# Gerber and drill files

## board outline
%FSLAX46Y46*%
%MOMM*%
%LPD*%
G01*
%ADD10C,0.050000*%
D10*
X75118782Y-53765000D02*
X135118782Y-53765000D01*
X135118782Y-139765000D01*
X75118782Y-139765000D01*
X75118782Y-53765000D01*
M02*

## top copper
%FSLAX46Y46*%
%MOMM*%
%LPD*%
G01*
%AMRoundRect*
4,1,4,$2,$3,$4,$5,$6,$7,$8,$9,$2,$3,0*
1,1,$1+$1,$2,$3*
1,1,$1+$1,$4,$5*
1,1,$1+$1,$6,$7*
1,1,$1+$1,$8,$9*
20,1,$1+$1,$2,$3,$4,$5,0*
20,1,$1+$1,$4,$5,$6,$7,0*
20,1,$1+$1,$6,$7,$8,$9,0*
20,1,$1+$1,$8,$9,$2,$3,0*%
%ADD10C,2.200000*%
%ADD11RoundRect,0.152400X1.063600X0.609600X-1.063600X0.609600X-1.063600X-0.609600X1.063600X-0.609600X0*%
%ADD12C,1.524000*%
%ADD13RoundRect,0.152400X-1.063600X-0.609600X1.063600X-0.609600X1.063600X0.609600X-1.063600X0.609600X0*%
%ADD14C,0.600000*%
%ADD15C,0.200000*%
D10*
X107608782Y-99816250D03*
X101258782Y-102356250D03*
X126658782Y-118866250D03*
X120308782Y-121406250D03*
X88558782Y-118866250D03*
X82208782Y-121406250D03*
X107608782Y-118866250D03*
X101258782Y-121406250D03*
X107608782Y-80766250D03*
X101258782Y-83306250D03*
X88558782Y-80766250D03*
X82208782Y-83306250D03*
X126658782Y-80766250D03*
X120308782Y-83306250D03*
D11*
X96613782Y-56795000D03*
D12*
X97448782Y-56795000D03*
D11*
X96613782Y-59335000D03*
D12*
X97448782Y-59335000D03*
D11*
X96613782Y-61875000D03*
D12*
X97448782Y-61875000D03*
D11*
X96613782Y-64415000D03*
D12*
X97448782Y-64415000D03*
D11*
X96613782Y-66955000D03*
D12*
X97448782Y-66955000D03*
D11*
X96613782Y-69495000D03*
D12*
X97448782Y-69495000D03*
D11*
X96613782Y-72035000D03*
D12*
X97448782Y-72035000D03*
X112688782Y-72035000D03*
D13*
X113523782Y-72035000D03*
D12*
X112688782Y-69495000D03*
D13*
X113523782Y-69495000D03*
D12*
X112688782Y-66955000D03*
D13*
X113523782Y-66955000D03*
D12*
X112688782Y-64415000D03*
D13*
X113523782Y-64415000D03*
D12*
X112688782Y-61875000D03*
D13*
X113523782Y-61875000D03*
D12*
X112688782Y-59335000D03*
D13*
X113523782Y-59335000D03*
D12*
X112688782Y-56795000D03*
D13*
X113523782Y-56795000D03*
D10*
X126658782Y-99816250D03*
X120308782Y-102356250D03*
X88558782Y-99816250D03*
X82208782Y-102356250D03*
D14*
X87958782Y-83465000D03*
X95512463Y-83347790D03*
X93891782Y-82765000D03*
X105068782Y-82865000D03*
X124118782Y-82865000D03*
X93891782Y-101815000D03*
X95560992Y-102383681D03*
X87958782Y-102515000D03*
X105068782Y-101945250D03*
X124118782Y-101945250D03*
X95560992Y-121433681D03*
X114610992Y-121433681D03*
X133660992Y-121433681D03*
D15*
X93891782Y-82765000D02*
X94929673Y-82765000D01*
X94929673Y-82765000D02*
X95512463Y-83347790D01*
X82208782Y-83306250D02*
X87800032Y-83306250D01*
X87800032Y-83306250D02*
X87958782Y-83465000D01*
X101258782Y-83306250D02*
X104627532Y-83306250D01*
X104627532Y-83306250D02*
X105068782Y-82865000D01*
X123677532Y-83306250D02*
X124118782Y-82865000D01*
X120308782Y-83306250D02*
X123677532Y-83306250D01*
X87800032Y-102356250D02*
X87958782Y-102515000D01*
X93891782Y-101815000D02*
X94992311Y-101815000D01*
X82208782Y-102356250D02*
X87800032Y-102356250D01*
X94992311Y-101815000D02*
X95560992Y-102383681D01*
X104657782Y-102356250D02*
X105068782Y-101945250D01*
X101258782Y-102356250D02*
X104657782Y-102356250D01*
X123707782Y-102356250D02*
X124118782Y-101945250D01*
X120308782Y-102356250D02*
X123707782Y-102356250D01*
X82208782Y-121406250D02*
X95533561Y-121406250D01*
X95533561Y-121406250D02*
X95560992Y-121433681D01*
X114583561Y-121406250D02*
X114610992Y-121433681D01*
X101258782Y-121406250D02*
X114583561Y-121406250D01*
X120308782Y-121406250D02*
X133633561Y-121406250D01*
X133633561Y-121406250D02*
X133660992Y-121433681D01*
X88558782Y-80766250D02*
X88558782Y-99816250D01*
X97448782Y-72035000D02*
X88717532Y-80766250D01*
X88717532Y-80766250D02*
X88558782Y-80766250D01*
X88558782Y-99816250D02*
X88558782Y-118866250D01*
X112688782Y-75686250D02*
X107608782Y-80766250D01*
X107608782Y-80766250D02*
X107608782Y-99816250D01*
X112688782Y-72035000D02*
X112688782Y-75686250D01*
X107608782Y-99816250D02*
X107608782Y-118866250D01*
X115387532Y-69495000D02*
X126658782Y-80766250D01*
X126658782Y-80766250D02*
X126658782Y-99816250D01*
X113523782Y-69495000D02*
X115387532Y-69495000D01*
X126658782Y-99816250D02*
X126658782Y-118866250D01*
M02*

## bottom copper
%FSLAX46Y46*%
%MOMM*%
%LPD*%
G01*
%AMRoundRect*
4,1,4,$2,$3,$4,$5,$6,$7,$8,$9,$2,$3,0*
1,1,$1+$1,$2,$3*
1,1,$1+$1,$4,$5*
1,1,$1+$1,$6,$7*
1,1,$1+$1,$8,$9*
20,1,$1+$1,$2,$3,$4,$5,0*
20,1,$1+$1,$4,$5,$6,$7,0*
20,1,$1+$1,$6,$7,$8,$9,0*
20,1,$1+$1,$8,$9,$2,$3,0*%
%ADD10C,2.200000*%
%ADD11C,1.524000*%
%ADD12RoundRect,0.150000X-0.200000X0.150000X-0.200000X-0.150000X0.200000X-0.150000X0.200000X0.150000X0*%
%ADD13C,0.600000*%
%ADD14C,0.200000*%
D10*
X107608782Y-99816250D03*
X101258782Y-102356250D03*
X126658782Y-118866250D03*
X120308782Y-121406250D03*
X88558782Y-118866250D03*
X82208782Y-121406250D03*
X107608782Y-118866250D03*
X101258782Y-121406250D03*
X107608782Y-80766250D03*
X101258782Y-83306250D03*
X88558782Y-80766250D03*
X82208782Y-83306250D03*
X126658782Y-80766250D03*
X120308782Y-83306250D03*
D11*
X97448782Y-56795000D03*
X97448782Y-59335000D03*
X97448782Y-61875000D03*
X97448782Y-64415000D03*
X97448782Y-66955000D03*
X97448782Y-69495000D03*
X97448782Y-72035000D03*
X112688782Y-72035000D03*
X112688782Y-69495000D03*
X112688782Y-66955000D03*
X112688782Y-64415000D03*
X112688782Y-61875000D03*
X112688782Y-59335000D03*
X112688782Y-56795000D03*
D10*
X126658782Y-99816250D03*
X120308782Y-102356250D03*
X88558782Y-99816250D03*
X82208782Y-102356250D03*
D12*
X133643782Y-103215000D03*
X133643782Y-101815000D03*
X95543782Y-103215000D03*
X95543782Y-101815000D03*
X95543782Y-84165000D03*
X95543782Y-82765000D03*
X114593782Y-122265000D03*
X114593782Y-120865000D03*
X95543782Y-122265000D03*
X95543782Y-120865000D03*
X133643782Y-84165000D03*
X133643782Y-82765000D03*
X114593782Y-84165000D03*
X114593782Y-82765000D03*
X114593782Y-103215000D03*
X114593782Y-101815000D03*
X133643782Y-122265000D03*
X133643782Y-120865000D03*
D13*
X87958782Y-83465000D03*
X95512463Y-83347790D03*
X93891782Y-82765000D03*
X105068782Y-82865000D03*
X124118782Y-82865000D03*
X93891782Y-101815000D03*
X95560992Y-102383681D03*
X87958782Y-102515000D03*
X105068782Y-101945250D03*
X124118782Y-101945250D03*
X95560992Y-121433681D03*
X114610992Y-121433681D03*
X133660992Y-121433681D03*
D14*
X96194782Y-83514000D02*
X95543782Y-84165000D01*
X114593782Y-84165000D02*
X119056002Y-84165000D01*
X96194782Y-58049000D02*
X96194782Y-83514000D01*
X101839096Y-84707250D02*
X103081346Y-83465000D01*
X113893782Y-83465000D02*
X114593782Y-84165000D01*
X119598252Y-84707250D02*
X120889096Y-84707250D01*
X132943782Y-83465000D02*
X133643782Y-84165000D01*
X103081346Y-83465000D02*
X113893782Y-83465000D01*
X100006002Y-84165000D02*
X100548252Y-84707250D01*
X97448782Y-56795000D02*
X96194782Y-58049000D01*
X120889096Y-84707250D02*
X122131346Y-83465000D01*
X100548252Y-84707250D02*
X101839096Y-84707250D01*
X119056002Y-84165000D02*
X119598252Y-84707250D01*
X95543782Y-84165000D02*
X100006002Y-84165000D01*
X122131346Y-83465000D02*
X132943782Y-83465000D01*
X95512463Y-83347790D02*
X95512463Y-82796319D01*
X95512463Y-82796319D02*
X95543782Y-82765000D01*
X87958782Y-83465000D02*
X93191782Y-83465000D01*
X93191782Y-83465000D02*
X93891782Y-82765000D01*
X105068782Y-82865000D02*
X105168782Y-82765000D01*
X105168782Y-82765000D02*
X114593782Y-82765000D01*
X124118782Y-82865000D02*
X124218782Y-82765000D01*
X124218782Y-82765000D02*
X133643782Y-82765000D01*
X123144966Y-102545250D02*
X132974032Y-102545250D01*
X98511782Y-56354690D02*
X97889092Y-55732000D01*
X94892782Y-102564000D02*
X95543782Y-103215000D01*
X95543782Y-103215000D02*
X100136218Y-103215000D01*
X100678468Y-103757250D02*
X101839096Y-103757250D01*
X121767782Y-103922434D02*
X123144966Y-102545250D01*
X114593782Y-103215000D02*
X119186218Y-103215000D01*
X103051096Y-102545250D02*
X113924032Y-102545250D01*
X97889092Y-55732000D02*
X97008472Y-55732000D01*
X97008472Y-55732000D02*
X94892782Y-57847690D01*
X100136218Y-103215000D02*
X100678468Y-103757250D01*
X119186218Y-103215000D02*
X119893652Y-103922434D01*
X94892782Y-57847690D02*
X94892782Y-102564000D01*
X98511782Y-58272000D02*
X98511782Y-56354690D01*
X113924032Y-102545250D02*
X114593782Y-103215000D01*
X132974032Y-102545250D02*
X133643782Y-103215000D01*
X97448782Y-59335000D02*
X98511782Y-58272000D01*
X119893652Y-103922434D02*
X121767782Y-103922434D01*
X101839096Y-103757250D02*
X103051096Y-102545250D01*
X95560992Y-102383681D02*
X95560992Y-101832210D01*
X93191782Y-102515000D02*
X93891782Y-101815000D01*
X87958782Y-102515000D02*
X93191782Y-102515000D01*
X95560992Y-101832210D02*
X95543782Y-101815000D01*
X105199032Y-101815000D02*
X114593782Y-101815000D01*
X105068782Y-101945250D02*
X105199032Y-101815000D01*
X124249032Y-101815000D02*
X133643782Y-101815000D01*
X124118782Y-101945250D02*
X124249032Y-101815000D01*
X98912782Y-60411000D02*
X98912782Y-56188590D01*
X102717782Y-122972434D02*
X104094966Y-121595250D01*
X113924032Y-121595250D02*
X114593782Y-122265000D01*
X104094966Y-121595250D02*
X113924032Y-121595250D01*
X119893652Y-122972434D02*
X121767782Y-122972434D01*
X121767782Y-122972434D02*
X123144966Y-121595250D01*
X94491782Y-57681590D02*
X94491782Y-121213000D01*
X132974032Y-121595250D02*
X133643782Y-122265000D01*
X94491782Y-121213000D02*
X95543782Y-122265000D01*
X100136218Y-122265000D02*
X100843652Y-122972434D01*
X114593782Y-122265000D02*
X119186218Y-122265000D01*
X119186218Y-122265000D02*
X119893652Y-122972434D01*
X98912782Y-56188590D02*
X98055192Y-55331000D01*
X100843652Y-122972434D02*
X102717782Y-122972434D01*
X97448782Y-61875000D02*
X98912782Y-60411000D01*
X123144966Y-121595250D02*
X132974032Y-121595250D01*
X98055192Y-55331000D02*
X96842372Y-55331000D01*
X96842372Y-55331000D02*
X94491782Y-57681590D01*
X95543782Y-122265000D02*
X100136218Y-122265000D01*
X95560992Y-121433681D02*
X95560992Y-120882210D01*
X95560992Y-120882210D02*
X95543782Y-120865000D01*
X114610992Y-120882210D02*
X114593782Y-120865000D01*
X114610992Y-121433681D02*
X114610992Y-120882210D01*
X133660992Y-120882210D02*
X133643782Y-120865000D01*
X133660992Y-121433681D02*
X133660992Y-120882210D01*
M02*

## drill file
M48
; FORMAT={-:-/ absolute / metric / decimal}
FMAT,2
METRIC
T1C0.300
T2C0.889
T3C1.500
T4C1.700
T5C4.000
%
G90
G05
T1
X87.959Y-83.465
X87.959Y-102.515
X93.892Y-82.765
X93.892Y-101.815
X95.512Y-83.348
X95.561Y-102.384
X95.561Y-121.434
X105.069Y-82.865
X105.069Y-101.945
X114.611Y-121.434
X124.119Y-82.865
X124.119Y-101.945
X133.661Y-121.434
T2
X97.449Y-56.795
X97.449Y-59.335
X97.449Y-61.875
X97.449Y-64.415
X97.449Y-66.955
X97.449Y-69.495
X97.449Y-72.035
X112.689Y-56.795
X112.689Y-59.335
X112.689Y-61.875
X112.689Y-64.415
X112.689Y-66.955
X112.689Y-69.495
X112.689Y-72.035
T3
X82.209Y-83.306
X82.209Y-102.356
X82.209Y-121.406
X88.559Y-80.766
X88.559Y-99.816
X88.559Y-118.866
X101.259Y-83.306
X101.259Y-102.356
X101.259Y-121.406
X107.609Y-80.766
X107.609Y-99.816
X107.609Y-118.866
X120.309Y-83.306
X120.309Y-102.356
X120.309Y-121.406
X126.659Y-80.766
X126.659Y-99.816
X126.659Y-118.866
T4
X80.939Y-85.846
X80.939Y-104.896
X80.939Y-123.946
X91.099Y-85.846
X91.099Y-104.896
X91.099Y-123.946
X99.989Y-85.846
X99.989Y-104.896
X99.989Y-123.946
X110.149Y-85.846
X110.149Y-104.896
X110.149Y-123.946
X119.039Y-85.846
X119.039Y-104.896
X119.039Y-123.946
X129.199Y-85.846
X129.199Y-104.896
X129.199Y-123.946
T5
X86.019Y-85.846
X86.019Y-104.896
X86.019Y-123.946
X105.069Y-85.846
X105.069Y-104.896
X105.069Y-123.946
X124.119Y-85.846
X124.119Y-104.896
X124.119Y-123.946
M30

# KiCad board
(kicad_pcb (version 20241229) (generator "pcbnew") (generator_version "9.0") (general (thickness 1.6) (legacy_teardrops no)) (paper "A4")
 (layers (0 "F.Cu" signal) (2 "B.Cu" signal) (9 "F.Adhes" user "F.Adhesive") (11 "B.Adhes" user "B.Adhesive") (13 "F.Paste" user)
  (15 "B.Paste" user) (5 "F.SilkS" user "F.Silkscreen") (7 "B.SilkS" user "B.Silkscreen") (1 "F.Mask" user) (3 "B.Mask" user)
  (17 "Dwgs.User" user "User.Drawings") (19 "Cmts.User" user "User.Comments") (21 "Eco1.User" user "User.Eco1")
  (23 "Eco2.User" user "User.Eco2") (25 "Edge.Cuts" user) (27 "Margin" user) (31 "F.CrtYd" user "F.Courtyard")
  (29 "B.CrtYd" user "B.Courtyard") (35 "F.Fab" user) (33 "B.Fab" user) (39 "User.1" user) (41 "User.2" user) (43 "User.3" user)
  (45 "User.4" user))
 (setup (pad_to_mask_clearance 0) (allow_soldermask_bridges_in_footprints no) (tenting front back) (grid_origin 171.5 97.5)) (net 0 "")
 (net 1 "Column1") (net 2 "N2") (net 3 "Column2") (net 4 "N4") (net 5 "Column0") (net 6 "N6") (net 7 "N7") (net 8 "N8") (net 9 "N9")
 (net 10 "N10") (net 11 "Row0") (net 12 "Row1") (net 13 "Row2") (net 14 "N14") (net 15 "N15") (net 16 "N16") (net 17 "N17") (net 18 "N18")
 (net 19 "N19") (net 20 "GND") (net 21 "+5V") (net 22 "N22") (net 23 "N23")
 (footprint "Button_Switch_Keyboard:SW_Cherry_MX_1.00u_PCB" (layer "F.Cu") (at 107.608782 99.81625)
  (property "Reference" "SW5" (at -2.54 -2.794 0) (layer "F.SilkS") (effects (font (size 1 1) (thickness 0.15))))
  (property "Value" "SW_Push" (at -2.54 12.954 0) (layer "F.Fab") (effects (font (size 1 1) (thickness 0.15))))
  (pad "" np_thru_hole circle (at -7.62 5.08) (size 1.7 1.7) (drill 1.7) (layers "*.Cu" "*.Mask"))
  (pad "" np_thru_hole circle (at -2.54 5.08) (size 4 4) (drill 4) (layers "*.Cu" "*.Mask"))
  (pad "" np_thru_hole circle (at 2.54 5.08) (size 1.7 1.7) (drill 1.7) (layers "*.Cu" "*.Mask"))
  (pad "1" thru_hole circle (at 0 0) (size 2.2 2.2) (drill 1.5) (layers "*.Cu" "*.Mask") (remove_unused_layers no) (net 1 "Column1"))
  (pad "2" thru_hole circle (at -6.35 2.54) (size 2.2 2.2) (drill 1.5) (layers "*.Cu" "*.Mask") (remove_unused_layers no) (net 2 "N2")))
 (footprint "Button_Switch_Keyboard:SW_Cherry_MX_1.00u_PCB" (layer "F.Cu") (at 126.658782 118.86625)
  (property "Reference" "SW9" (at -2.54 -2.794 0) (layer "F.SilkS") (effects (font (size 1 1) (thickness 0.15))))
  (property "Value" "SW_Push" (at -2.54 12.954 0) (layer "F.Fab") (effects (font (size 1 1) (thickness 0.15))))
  (pad "" np_thru_hole circle (at -7.62 5.08) (size 1.7 1.7) (drill 1.7) (layers "*.Cu" "*.Mask"))
  (pad "" np_thru_hole circle (at -2.54 5.08) (size 4 4) (drill 4) (layers "*.Cu" "*.Mask"))
  (pad "" np_thru_hole circle (at 2.54 5.08) (size 1.7 1.7) (drill 1.7) (layers "*.Cu" "*.Mask"))
  (pad "1" thru_hole circle (at 0 0) (size 2.2 2.2) (drill 1.5) (layers "*.Cu" "*.Mask") (remove_unused_layers no) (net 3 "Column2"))
  (pad "2" thru_hole circle (at -6.35 2.54) (size 2.2 2.2) (drill 1.5) (layers "*.Cu" "*.Mask") (remove_unused_layers no) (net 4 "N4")))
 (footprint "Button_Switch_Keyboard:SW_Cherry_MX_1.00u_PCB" (layer "F.Cu") (at 88.558782 118.86625)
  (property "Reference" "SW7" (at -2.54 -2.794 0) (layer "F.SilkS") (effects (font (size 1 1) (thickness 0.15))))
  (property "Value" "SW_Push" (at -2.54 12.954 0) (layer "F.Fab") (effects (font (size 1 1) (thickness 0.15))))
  (pad "" np_thru_hole circle (at -7.62 5.08) (size 1.7 1.7) (drill 1.7) (layers "*.Cu" "*.Mask"))
  (pad "" np_thru_hole circle (at -2.54 5.08) (size 4 4) (drill 4) (layers "*.Cu" "*.Mask"))
  (pad "" np_thru_hole circle (at 2.54 5.08) (size 1.7 1.7) (drill 1.7) (layers "*.Cu" "*.Mask"))
  (pad "1" thru_hole circle (at 0 0) (size 2.2 2.2) (drill 1.5) (layers "*.Cu" "*.Mask") (remove_unused_layers no) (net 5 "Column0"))
  (pad "2" thru_hole circle (at -6.35 2.54) (size 2.2 2.2) (drill 1.5) (layers "*.Cu" "*.Mask") (remove_unused_layers no) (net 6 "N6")))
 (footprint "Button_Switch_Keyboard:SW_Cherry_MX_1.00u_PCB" (layer "F.Cu") (at 107.608782 118.86625)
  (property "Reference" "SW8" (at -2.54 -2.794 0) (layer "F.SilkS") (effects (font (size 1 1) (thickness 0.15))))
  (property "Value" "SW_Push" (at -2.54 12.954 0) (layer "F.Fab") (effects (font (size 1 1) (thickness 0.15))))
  (pad "" np_thru_hole circle (at -7.62 5.08) (size 1.7 1.7) (drill 1.7) (layers "*.Cu" "*.Mask"))
  (pad "" np_thru_hole circle (at -2.54 5.08) (size 4 4) (drill 4) (layers "*.Cu" "*.Mask"))
  (pad "" np_thru_hole circle (at 2.54 5.08) (size 1.7 1.7) (drill 1.7) (layers "*.Cu" "*.Mask"))
  (pad "1" thru_hole circle (at 0 0) (size 2.2 2.2) (drill 1.5) (layers "*.Cu" "*.Mask") (remove_unused_layers no) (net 1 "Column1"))
  (pad "2" thru_hole circle (at -6.35 2.54) (size 2.2 2.2) (drill 1.5) (layers "*.Cu" "*.Mask") (remove_unused_layers no) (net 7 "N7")))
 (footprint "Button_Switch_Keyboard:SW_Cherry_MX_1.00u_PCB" (layer "F.Cu") (at 107.608782 80.76625)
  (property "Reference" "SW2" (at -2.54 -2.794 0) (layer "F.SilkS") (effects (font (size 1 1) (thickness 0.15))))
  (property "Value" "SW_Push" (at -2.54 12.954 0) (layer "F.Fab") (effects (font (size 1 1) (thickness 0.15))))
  (pad "" np_thru_hole circle (at -7.62 5.08) (size 1.7 1.7) (drill 1.7) (layers "*.Cu" "*.Mask"))
  (pad "" np_thru_hole circle (at -2.54 5.08) (size 4 4) (drill 4) (layers "*.Cu" "*.Mask"))
  (pad "" np_thru_hole circle (at 2.54 5.08) (size 1.7 1.7) (drill 1.7) (layers "*.Cu" "*.Mask"))
  (pad "1" thru_hole circle (at 0 0) (size 2.2 2.2) (drill 1.5) (layers "*.Cu" "*.Mask") (remove_unused_layers no) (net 1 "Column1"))
  (pad "2" thru_hole circle (at -6.35 2.54) (size 2.2 2.2) (drill 1.5) (layers "*.Cu" "*.Mask") (remove_unused_layers no) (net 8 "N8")))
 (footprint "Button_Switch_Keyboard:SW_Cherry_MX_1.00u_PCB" (layer "F.Cu") (at 88.558782 80.76625)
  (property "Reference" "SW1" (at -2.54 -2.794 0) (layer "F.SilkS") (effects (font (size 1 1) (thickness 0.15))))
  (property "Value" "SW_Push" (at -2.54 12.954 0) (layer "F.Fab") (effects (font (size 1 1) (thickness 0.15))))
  (pad "" np_thru_hole circle (at -7.62 5.08) (size 1.7 1.7) (drill 1.7) (layers "*.Cu" "*.Mask"))
  (pad "" np_thru_hole circle (at -2.54 5.08) (size 4 4) (drill 4) (layers "*.Cu" "*.Mask"))
  (pad "" np_thru_hole circle (at 2.54 5.08) (size 1.7 1.7) (drill 1.7) (layers "*.Cu" "*.Mask"))
  (pad "1" thru_hole circle (at 0 0) (size 2.2 2.2) (drill 1.5) (layers "*.Cu" "*.Mask") (remove_unused_layers no) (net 5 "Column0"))
  (pad "2" thru_hole circle (at -6.35 2.54) (size 2.2 2.2) (drill 1.5) (layers "*.Cu" "*.Mask") (remove_unused_layers no) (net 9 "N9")))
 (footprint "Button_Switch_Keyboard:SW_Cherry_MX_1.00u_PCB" (layer "F.Cu") (at 126.658782 80.76625)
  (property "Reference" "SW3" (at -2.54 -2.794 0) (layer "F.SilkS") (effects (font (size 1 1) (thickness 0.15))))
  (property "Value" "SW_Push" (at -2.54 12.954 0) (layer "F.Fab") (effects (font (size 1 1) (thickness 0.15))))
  (pad "" np_thru_hole circle (at -7.62 5.08) (size 1.7 1.7) (drill 1.7) (layers "*.Cu" "*.Mask"))
  (pad "" np_thru_hole circle (at -2.54 5.08) (size 4 4) (drill 4) (layers "*.Cu" "*.Mask"))
  (pad "" np_thru_hole circle (at 2.54 5.08) (size 1.7 1.7) (drill 1.7) (layers "*.Cu" "*.Mask"))
  (pad "1" thru_hole circle (at 0 0) (size 2.2 2.2) (drill 1.5) (layers "*.Cu" "*.Mask") (remove_unused_layers no) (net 3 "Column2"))
  (pad "2" thru_hole circle (at -6.35 2.54) (size 2.2 2.2) (drill 1.5) (layers "*.Cu" "*.Mask") (remove_unused_layers no) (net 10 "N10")))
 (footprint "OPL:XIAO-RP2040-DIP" (layer "F.Cu") (at 105.068782 64.415)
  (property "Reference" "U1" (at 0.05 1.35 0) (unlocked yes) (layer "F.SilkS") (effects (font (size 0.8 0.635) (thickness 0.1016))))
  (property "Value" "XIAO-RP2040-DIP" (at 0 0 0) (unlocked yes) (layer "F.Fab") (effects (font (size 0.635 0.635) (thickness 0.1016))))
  (pad "1" smd roundrect (at -8.455 -7.62 180) (size 2.432 1.524) (layers "F.Cu" "F.Mask") (roundrect_rratio 0.1) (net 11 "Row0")
   (thermal_bridge_angle 45))
  (pad "1" thru_hole circle (at -7.62 -7.62 180) (size 1.524 1.524) (drill 0.889) (layers "*.Cu" "*.Mask") (remove_unused_layers no)
   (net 11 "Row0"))
  (pad "2" smd roundrect (at -8.455 -5.08 180) (size 2.432 1.524) (layers "F.Cu" "F.Mask") (roundrect_rratio 0.1) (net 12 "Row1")
   (thermal_bridge_angle 45))
  (pad "2" thru_hole circle (at -7.62 -5.08 180) (size 1.524 1.524) (drill 0.889) (layers "*.Cu" "*.Mask") (remove_unused_layers no)
   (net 12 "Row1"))
  (pad "3" smd roundrect (at -8.455 -2.54 180) (size 2.432 1.524) (layers "F.Cu" "F.Mask") (roundrect_rratio 0.1) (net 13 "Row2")
   (thermal_bridge_angle 45))
  (pad "3" thru_hole circle (at -7.62 -2.54 180) (size 1.524 1.524) (drill 0.889) (layers "*.Cu" "*.Mask") (remove_unused_layers no)
   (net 13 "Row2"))
  (pad "4" smd roundrect (at -8.455 0 180) (size 2.432 1.524) (layers "F.Cu" "F.Mask") (roundrect_rratio 0.1) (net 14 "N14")
   (thermal_bridge_angle 45))
  (pad "4" thru_hole circle (at -7.62 0 180) (size 1.524 1.524) (drill 0.889) (layers "*.Cu" "*.Mask") (remove_unused_layers no)
   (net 14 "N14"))
  (pad "5" smd roundrect (at -8.455 2.54 180) (size 2.432 1.524) (layers "F.Cu" "F.Mask") (roundrect_rratio 0.1) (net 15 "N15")
   (thermal_bridge_angle 45))
  (pad "5" thru_hole circle (at -7.62 2.54 180) (size 1.524 1.524) (drill 0.889) (layers "*.Cu" "*.Mask") (remove_unused_layers no)
   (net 15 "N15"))
  (pad "6" smd roundrect (at -8.455 5.08 180) (size 2.432 1.524) (layers "F.Cu" "F.Mask") (roundrect_rratio 0.1) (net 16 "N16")
   (thermal_bridge_angle 45))
  (pad "6" thru_hole circle (at -7.62 5.08 180) (size 1.524 1.524) (drill 0.889) (layers "*.Cu" "*.Mask") (remove_unused_layers no)
   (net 16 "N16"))
  (pad "7" smd roundrect (at -8.455 7.62 180) (size 2.432 1.524) (layers "F.Cu" "F.Mask") (roundrect_rratio 0.1) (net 5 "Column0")
   (thermal_bridge_angle 45))
  (pad "7" thru_hole circle (at -7.62 7.62 180) (size 1.524 1.524) (drill 0.889) (layers "*.Cu" "*.Mask") (remove_unused_layers no)
   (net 5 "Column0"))
  (pad "8" thru_hole circle (at 7.62 7.62) (size 1.524 1.524) (drill 0.889) (layers "*.Cu" "*.Mask") (remove_unused_layers no)
   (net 1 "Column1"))
  (pad "8" smd roundrect (at 8.455 7.62) (size 2.432 1.524) (layers "F.Cu" "F.Mask") (roundrect_rratio 0.1) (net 1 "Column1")
   (thermal_bridge_angle 45))
  (pad "9" thru_hole circle (at 7.62 5.08) (size 1.524 1.524) (drill 0.889) (layers "*.Cu" "*.Mask") (remove_unused_layers no)
   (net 3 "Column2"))
  (pad "9" smd roundrect (at 8.455 5.08) (size 2.432 1.524) (layers "F.Cu" "F.Mask") (roundrect_rratio 0.1) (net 3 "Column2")
   (thermal_bridge_angle 45))
  (pad "10" thru_hole circle (at 7.62 2.54) (size 1.524 1.524) (drill 0.889) (layers "*.Cu" "*.Mask") (remove_unused_layers no)
   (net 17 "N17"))
  (pad "10" smd roundrect (at 8.455 2.54) (size 2.432 1.524) (layers "F.Cu" "F.Mask") (roundrect_rratio 0.1) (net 17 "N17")
   (thermal_bridge_angle 45))
  (pad "11" thru_hole circle (at 7.62 0) (size 1.524 1.524) (drill 0.889) (layers "*.Cu" "*.Mask") (remove_unused_layers no) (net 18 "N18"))
  (pad "11" smd roundrect (at 8.455 0) (size 2.432 1.524) (layers "F.Cu" "F.Mask") (roundrect_rratio 0.1) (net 18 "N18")
   (thermal_bridge_angle 45))
  (pad "12" thru_hole circle (at 7.62 -2.54) (size 1.524 1.524) (drill 0.889) (layers "*.Cu" "*.Mask") (remove_unused_layers no)
   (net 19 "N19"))
  (pad "12" smd roundrect (at 8.455 -2.54) (size 2.432 1.524) (layers "F.Cu" "F.Mask") (roundrect_rratio 0.1) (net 19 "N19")
   (thermal_bridge_angle 45))
  (pad "13" thru_hole circle (at 7.62 -5.08) (size 1.524 1.524) (drill 0.889) (layers "*.Cu" "*.Mask") (remove_unused_layers no)
   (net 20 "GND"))
  (pad "13" smd roundrect (at 8.455 -5.08) (size 2.432 1.524) (layers "F.Cu" "F.Mask") (roundrect_rratio 0.1) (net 20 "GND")
   (thermal_bridge_angle 45))
  (pad "14" thru_hole circle (at 7.62 -7.62) (size 1.524 1.524) (drill 0.889) (layers "*.Cu" "*.Mask") (remove_unused_layers no)
   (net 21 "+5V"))
  (pad "14" smd roundrect (at 8.455 -7.62) (size 2.432 1.524) (layers "F.Cu" "F.Mask") (roundrect_rratio 0.1) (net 21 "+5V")
   (thermal_bridge_angle 45)))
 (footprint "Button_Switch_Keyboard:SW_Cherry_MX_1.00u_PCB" (layer "F.Cu") (at 126.658782 99.81625)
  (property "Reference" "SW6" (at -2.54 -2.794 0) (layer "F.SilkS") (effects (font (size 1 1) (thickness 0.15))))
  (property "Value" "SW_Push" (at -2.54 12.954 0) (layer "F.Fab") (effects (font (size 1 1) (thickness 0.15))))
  (pad "" np_thru_hole circle (at -7.62 5.08) (size 1.7 1.7) (drill 1.7) (layers "*.Cu" "*.Mask"))
  (pad "" np_thru_hole circle (at -2.54 5.08) (size 4 4) (drill 4) (layers "*.Cu" "*.Mask"))
  (pad "" np_thru_hole circle (at 2.54 5.08) (size 1.7 1.7) (drill 1.7) (layers "*.Cu" "*.Mask"))
  (pad "1" thru_hole circle (at 0 0) (size 2.2 2.2) (drill 1.5) (layers "*.Cu" "*.Mask") (remove_unused_layers no) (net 3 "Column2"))
  (pad "2" thru_hole circle (at -6.35 2.54) (size 2.2 2.2) (drill 1.5) (layers "*.Cu" "*.Mask") (remove_unused_layers no) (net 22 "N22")))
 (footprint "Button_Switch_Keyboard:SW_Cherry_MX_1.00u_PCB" (layer "F.Cu") (at 88.558782 99.81625)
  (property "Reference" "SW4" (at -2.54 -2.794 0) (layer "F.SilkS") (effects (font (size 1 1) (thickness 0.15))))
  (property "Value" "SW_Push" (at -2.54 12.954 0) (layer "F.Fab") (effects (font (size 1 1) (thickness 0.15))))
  (pad "" np_thru_hole circle (at -7.62 5.08) (size 1.7 1.7) (drill 1.7) (layers "*.Cu" "*.Mask"))
  (pad "" np_thru_hole circle (at -2.54 5.08) (size 4 4) (drill 4) (layers "*.Cu" "*.Mask"))
  (pad "" np_thru_hole circle (at 2.54 5.08) (size 1.7 1.7) (drill 1.7) (layers "*.Cu" "*.Mask"))
  (pad "1" thru_hole circle (at 0 0) (size 2.2 2.2) (drill 1.5) (layers "*.Cu" "*.Mask") (remove_unused_layers no) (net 5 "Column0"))
  (pad "2" thru_hole circle (at -6.35 2.54) (size 2.2 2.2) (drill 1.5) (layers "*.Cu" "*.Mask") (remove_unused_layers no) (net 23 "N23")))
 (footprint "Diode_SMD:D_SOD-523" (layer "B.Cu") (at 133.643782 102.515 90)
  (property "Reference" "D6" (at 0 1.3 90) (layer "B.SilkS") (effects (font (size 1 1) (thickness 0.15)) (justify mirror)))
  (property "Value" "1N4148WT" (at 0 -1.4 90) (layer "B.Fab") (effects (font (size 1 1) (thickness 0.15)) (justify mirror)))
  (pad "1" smd roundrect (at -0.7 0 270) (size 0.6 0.7) (layers "B.Cu" "B.Mask" "B.Paste") (roundrect_rratio 0.25) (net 12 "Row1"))
  (pad "2" smd roundrect (at 0.7 0 270) (size 0.6 0.7) (layers "B.Cu" "B.Mask" "B.Paste") (roundrect_rratio 0.25) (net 22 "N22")))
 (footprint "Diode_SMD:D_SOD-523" (layer "B.Cu") (at 95.543782 102.515 90)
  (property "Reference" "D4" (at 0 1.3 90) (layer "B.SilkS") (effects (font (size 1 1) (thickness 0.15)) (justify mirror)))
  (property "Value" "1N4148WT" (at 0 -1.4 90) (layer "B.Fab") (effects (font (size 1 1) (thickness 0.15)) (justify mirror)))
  (pad "1" smd roundrect (at -0.7 0 270) (size 0.6 0.7) (layers "B.Cu" "B.Mask" "B.Paste") (roundrect_rratio 0.25) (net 12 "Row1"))
  (pad "2" smd roundrect (at 0.7 0 270) (size 0.6 0.7) (layers "B.Cu" "B.Mask" "B.Paste") (roundrect_rratio 0.25) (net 23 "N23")))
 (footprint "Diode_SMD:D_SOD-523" (layer "B.Cu") (at 95.543782 83.465 90)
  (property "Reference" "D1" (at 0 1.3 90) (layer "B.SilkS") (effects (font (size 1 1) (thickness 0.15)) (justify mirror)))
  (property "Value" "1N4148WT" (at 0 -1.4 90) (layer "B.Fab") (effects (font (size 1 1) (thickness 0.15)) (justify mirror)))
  (pad "1" smd roundrect (at -0.7 0 270) (size 0.6 0.7) (layers "B.Cu" "B.Mask" "B.Paste") (roundrect_rratio 0.25) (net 11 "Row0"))
  (pad "2" smd roundrect (at 0.7 0 270) (size 0.6 0.7) (layers "B.Cu" "B.Mask" "B.Paste") (roundrect_rratio 0.25) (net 9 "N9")))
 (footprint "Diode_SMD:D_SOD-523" (layer "B.Cu") (at 114.593782 121.565 90)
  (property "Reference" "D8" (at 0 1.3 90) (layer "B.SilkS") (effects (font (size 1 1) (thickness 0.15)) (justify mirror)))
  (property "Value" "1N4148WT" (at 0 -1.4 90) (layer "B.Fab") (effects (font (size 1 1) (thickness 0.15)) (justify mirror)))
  (pad "1" smd roundrect (at -0.7 0 270) (size 0.6 0.7) (layers "B.Cu" "B.Mask" "B.Paste") (roundrect_rratio 0.25) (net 13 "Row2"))
  (pad "2" smd roundrect (at 0.7 0 270) (size 0.6 0.7) (layers "B.Cu" "B.Mask" "B.Paste") (roundrect_rratio 0.25) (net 7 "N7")))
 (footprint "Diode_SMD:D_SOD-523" (layer "B.Cu") (at 95.543782 121.565 90)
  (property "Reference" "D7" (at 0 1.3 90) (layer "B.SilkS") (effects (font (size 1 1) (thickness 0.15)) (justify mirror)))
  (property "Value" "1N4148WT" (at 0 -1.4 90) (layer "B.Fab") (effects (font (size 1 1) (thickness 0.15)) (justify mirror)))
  (pad "1" smd roundrect (at -0.7 0 270) (size 0.6 0.7) (layers "B.Cu" "B.Mask" "B.Paste") (roundrect_rratio 0.25) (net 13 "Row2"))
  (pad "2" smd roundrect (at 0.7 0 270) (size 0.6 0.7) (layers "B.Cu" "B.Mask" "B.Paste") (roundrect_rratio 0.25) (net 6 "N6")))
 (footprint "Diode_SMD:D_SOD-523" (layer "B.Cu") (at 133.643782 83.465 90)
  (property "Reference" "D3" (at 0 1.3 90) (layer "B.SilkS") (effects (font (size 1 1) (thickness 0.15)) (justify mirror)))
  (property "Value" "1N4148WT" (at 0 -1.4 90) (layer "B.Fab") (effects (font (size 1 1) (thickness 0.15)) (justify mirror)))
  (pad "1" smd roundrect (at -0.7 0 270) (size 0.6 0.7) (layers "B.Cu" "B.Mask" "B.Paste") (roundrect_rratio 0.25) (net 11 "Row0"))
  (pad "2" smd roundrect (at 0.7 0 270) (size 0.6 0.7) (layers "B.Cu" "B.Mask" "B.Paste") (roundrect_rratio 0.25) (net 10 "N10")))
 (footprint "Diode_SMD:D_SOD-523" (layer "B.Cu") (at 114.593782 83.465 90)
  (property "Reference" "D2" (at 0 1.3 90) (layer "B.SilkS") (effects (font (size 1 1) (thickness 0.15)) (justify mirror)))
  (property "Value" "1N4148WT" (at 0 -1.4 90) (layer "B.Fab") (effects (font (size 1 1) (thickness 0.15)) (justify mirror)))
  (pad "1" smd roundrect (at -0.7 0 270) (size 0.6 0.7) (layers "B.Cu" "B.Mask" "B.Paste") (roundrect_rratio 0.25) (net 11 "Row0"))
  (pad "2" smd roundrect (at 0.7 0 270) (size 0.6 0.7) (layers "B.Cu" "B.Mask" "B.Paste") (roundrect_rratio 0.25) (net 8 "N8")))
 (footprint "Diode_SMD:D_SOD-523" (layer "B.Cu") (at 114.593782 102.515 90)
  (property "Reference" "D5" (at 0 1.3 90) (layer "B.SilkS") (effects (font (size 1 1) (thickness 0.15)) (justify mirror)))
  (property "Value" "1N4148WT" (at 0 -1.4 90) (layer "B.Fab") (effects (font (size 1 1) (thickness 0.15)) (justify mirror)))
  (pad "1" smd roundrect (at -0.7 0 270) (size 0.6 0.7) (layers "B.Cu" "B.Mask" "B.Paste") (roundrect_rratio 0.25) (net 12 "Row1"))
  (pad "2" smd roundrect (at 0.7 0 270) (size 0.6 0.7) (layers "B.Cu" "B.Mask" "B.Paste") (roundrect_rratio 0.25) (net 2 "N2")))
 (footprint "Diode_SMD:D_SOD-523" (layer "B.Cu") (at 133.643782 121.565 90)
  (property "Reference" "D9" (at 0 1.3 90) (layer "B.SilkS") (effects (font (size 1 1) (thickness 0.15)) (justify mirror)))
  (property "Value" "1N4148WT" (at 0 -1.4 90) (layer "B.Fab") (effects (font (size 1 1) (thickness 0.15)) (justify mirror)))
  (pad "1" smd roundrect (at -0.7 0 270) (size 0.6 0.7) (layers "B.Cu" "B.Mask" "B.Paste") (roundrect_rratio 0.25) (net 13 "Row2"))
  (pad "2" smd roundrect (at 0.7 0 270) (size 0.6 0.7) (layers "B.Cu" "B.Mask" "B.Paste") (roundrect_rratio 0.25) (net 4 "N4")))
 (gr_rect (start 75.118782 53.765) (end 135.118782 139.765) (stroke (width 0.05) (type default)) (fill no) (layer "Edge.Cuts"))
 (segment (start 96.194782 83.514) (end 95.543782 84.165) (width 0.2) (layer "B.Cu") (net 11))
 (segment (start 114.593782 84.165) (end 119.056002 84.165) (width 0.2) (layer "B.Cu") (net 11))
 (segment (start 96.194782 58.049) (end 96.194782 83.514) (width 0.2) (layer "B.Cu") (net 11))
 (segment (start 101.839096 84.70725) (end 103.081346 83.465) (width 0.2) (layer "B.Cu") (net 11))
 (segment (start 113.893782 83.465) (end 114.593782 84.165) (width 0.2) (layer "B.Cu") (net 11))
 (segment (start 119.598252 84.70725) (end 120.889096 84.70725) (width 0.2) (layer "B.Cu") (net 11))
 (segment (start 132.943782 83.465) (end 133.643782 84.165) (width 0.2) (layer "B.Cu") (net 11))
 (segment (start 103.081346 83.465) (end 113.893782 83.465) (width 0.2) (layer "B.Cu") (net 11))
 (segment (start 100.006002 84.165) (end 100.548252 84.70725) (width 0.2) (layer "B.Cu") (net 11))
 (segment (start 97.448782 56.795) (end 96.194782 58.049) (width 0.2) (layer "B.Cu") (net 11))
 (segment (start 120.889096 84.70725) (end 122.131346 83.465) (width 0.2) (layer "B.Cu") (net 11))
 (segment (start 100.548252 84.70725) (end 101.839096 84.70725) (width 0.2) (layer "B.Cu") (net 11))
 (segment (start 119.056002 84.165) (end 119.598252 84.70725) (width 0.2) (layer "B.Cu") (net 11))
 (segment (start 95.543782 84.165) (end 100.006002 84.165) (width 0.2) (layer "B.Cu") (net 11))
 (segment (start 122.131346 83.465) (end 132.943782 83.465) (width 0.2) (layer "B.Cu") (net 11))
 (segment (start 93.891782 82.765) (end 94.929673 82.765) (width 0.2) (layer "F.Cu") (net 9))
 (segment (start 94.929673 82.765) (end 95.512463 83.34779) (width 0.2) (layer "F.Cu") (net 9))
 (segment (start 82.208782 83.30625) (end 87.800032 83.30625) (width 0.2) (layer "F.Cu") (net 9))
 (segment (start 87.800032 83.30625) (end 87.958782 83.465) (width 0.2) (layer "F.Cu") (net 9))
 (via (at 87.958782 83.465) (size 0.6) (drill 0.3) (layers "F.Cu" "B.Cu") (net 9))
 (via (at 95.512463 83.34779) (size 0.6) (drill 0.3) (layers "F.Cu" "B.Cu") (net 9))
 (via (at 93.891782 82.765) (size 0.6) (drill 0.3) (layers "F.Cu" "B.Cu") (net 9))
 (segment (start 95.512463 83.34779) (end 95.512463 82.796319) (width 0.2) (layer "B.Cu") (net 9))
 (segment (start 95.512463 82.796319) (end 95.543782 82.765) (width 0.2) (layer "B.Cu") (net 9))
 (segment (start 87.958782 83.465) (end 93.191782 83.465) (width 0.2) (layer "B.Cu") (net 9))
 (segment (start 93.191782 83.465) (end 93.891782 82.765) (width 0.2) (layer "B.Cu") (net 9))
 (segment (start 101.258782 83.30625) (end 104.627532 83.30625) (width 0.2) (layer "F.Cu") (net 8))
 (segment (start 104.627532 83.30625) (end 105.068782 82.865) (width 0.2) (layer "F.Cu") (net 8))
 (via (at 105.068782 82.865) (size 0.6) (drill 0.3) (layers "F.Cu" "B.Cu") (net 8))
 (segment (start 105.068782 82.865) (end 105.168782 82.765) (width 0.2) (layer "B.Cu") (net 8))
 (segment (start 105.168782 82.765) (end 114.593782 82.765) (width 0.2) (layer "B.Cu") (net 8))
 (segment (start 123.677532 83.30625) (end 124.118782 82.865) (width 0.2) (layer "F.Cu") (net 10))
 (segment (start 120.308782 83.30625) (end 123.677532 83.30625) (width 0.2) (layer "F.Cu") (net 10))
 (via (at 124.118782 82.865) (size 0.6) (drill 0.3) (layers "F.Cu" "B.Cu") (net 10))
 (segment (start 124.118782 82.865) (end 124.218782 82.765) (width 0.2) (layer "B.Cu") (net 10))
 (segment (start 124.218782 82.765) (end 133.643782 82.765) (width 0.2) (layer "B.Cu") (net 10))
 (segment (start 123.144966 102.54525) (end 132.974032 102.54525) (width 0.2) (layer "B.Cu") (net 12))
 (segment (start 98.511782 56.35469) (end 97.889092 55.732) (width 0.2) (layer "B.Cu") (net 12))
 (segment (start 94.892782 102.564) (end 95.543782 103.215) (width 0.2) (layer "B.Cu") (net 12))
 (segment (start 95.543782 103.215) (end 100.136218 103.215) (width 0.2) (layer "B.Cu") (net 12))
 (segment (start 100.678468 103.75725) (end 101.839096 103.75725) (width 0.2) (layer "B.Cu") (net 12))
 (segment (start 121.767782 103.922434) (end 123.144966 102.54525) (width 0.2) (layer "B.Cu") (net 12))
 (segment (start 114.593782 103.215) (end 119.186218 103.215) (width 0.2) (layer "B.Cu") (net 12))
 (segment (start 103.051096 102.54525) (end 113.924032 102.54525) (width 0.2) (layer "B.Cu") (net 12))
 (segment (start 97.889092 55.732) (end 97.008472 55.732) (width 0.2) (layer "B.Cu") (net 12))
 (segment (start 97.008472 55.732) (end 94.892782 57.84769) (width 0.2) (layer "B.Cu") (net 12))
 (segment (start 100.136218 103.215) (end 100.678468 103.75725) (width 0.2) (layer "B.Cu") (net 12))
 (segment (start 119.186218 103.215) (end 119.893652 103.922434) (width 0.2) (layer "B.Cu") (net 12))
 (segment (start 94.892782 57.84769) (end 94.892782 102.564) (width 0.2) (layer "B.Cu") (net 12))
 (segment (start 98.511782 58.272) (end 98.511782 56.35469) (width 0.2) (layer "B.Cu") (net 12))
 (segment (start 113.924032 102.54525) (end 114.593782 103.215) (width 0.2) (layer "B.Cu") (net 12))
 (segment (start 132.974032 102.54525) (end 133.643782 103.215) (width 0.2) (layer "B.Cu") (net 12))
 (segment (start 97.448782 59.335) (end 98.511782 58.272) (width 0.2) (layer "B.Cu") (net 12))
 (segment (start 119.893652 103.922434) (end 121.767782 103.922434) (width 0.2) (layer "B.Cu") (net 12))
 (segment (start 101.839096 103.75725) (end 103.051096 102.54525) (width 0.2) (layer "B.Cu") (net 12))
 (segment (start 87.800032 102.35625) (end 87.958782 102.515) (width 0.2) (layer "F.Cu") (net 23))
 (segment (start 93.891782 101.815) (end 94.992311 101.815) (width 0.2) (layer "F.Cu") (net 23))
 (segment (start 82.208782 102.35625) (end 87.800032 102.35625) (width 0.2) (layer "F.Cu") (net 23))
 (segment (start 94.992311 101.815) (end 95.560992 102.383681) (width 0.2) (layer "F.Cu") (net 23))
 (via (at 93.891782 101.815) (size 0.6) (drill 0.3) (layers "F.Cu" "B.Cu") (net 23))
 (via (at 95.560992 102.383681) (size 0.6) (drill 0.3) (layers "F.Cu" "B.Cu") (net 23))
 (via (at 87.958782 102.515) (size 0.6) (drill 0.3) (layers "F.Cu" "B.Cu") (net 23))
 (segment (start 95.560992 102.383681) (end 95.560992 101.83221) (width 0.2) (layer "B.Cu") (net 23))
 (segment (start 93.191782 102.515) (end 93.891782 101.815) (width 0.2) (layer "B.Cu") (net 23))
 (segment (start 87.958782 102.515) (end 93.191782 102.515) (width 0.2) (layer "B.Cu") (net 23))
 (segment (start 95.560992 101.83221) (end 95.543782 101.815) (width 0.2) (layer "B.Cu") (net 23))
 (segment (start 104.657782 102.35625) (end 105.068782 101.94525) (width 0.2) (layer "F.Cu") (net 2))
 (segment (start 101.258782 102.35625) (end 104.657782 102.35625) (width 0.2) (layer "F.Cu") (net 2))
 (via (at 105.068782 101.94525) (size 0.6) (drill 0.3) (layers "F.Cu" "B.Cu") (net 2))
 (segment (start 105.199032 101.815) (end 114.593782 101.815) (width 0.2) (layer "B.Cu") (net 2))
 (segment (start 105.068782 101.94525) (end 105.199032 101.815) (width 0.2) (layer "B.Cu") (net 2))
 (segment (start 123.707782 102.35625) (end 124.118782 101.94525) (width 0.2) (layer "F.Cu") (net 22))
 (segment (start 120.308782 102.35625) (end 123.707782 102.35625) (width 0.2) (layer "F.Cu") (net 22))
 (via (at 124.118782 101.94525) (size 0.6) (drill 0.3) (layers "F.Cu" "B.Cu") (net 22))
 (segment (start 124.249032 101.815) (end 133.643782 101.815) (width 0.2) (layer "B.Cu") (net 22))
 (segment (start 124.118782 101.94525) (end 124.249032 101.815) (width 0.2) (layer "B.Cu") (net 22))
 (segment (start 98.912782 60.411) (end 98.912782 56.18859) (width 0.2) (layer "B.Cu") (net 13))
 (segment (start 102.717782 122.972434) (end 104.094966 121.59525) (width 0.2) (layer "B.Cu") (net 13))
 (segment (start 113.924032 121.59525) (end 114.593782 122.265) (width 0.2) (layer "B.Cu") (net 13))
 (segment (start 104.094966 121.59525) (end 113.924032 121.59525) (width 0.2) (layer "B.Cu") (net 13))
 (segment (start 119.893652 122.972434) (end 121.767782 122.972434) (width 0.2) (layer "B.Cu") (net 13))
 (segment (start 121.767782 122.972434) (end 123.144966 121.59525) (width 0.2) (layer "B.Cu") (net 13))
 (segment (start 94.491782 57.68159) (end 94.491782 121.213) (width 0.2) (layer "B.Cu") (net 13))
 (segment (start 132.974032 121.59525) (end 133.643782 122.265) (width 0.2) (layer "B.Cu") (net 13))
 (segment (start 94.491782 121.213) (end 95.543782 122.265) (width 0.2) (layer "B.Cu") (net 13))
 (segment (start 100.136218 122.265) (end 100.843652 122.972434) (width 0.2) (layer "B.Cu") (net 13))
 (segment (start 114.593782 122.265) (end 119.186218 122.265) (width 0.2) (layer "B.Cu") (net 13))
 (segment (start 119.186218 122.265) (end 119.893652 122.972434) (width 0.2) (layer "B.Cu") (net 13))
 (segment (start 98.912782 56.18859) (end 98.055192 55.331) (width 0.2) (layer "B.Cu") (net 13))
 (segment (start 100.843652 122.972434) (end 102.717782 122.972434) (width 0.2) (layer "B.Cu") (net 13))
 (segment (start 97.448782 61.875) (end 98.912782 60.411) (width 0.2) (layer "B.Cu") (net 13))
 (segment (start 123.144966 121.59525) (end 132.974032 121.59525) (width 0.2) (layer "B.Cu") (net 13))
 (segment (start 98.055192 55.331) (end 96.842372 55.331) (width 0.2) (layer "B.Cu") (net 13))
 (segment (start 96.842372 55.331) (end 94.491782 57.68159) (width 0.2) (layer "B.Cu") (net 13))
 (segment (start 95.543782 122.265) (end 100.136218 122.265) (width 0.2) (layer "B.Cu") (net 13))
 (segment (start 82.208782 121.40625) (end 95.533561 121.40625) (width 0.2) (layer "F.Cu") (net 6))
 (segment (start 95.533561 121.40625) (end 95.560992 121.433681) (width 0.2) (layer "F.Cu") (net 6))
 (via (at 95.560992 121.433681) (size 0.6) (drill 0.3) (layers "F.Cu" "B.Cu") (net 6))
 (segment (start 95.560992 121.433681) (end 95.560992 120.88221) (width 0.2) (layer "B.Cu") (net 6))
 (segment (start 95.560992 120.88221) (end 95.543782 120.865) (width 0.2) (layer "B.Cu") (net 6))
 (segment (start 114.583561 121.40625) (end 114.610992 121.433681) (width 0.2) (layer "F.Cu") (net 7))
 (segment (start 101.258782 121.40625) (end 114.583561 121.40625) (width 0.2) (layer "F.Cu") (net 7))
 (via (at 114.610992 121.433681) (size 0.6) (drill 0.3) (layers "F.Cu" "B.Cu") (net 7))
 (segment (start 114.610992 120.88221) (end 114.593782 120.865) (width 0.2) (layer "B.Cu") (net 7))
 (segment (start 114.610992 121.433681) (end 114.610992 120.88221) (width 0.2) (layer "B.Cu") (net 7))
 (segment (start 120.308782 121.40625) (end 133.633561 121.40625) (width 0.2) (layer "F.Cu") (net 4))
 (segment (start 133.633561 121.40625) (end 133.660992 121.433681) (width 0.2) (layer "F.Cu") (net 4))
 (via (at 133.660992 121.433681) (size 0.6) (drill 0.3) (layers "F.Cu" "B.Cu") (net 4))
 (segment (start 133.660992 120.88221) (end 133.643782 120.865) (width 0.2) (layer "B.Cu") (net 4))
 (segment (start 133.660992 121.433681) (end 133.660992 120.88221) (width 0.2) (layer "B.Cu") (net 4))
 (segment (start 88.558782 80.76625) (end 88.558782 99.81625) (width 0.2) (layer "F.Cu") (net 5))
 (segment (start 97.448782 72.035) (end 88.717532 80.76625) (width 0.2) (layer "F.Cu") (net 5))
 (segment (start 88.717532 80.76625) (end 88.558782 80.76625) (width 0.2) (layer "F.Cu") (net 5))
 (segment (start 88.558782 99.81625) (end 88.558782 118.86625) (width 0.2) (layer "F.Cu") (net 5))
 (segment (start 112.688782 75.68625) (end 107.608782 80.76625) (width 0.2) (layer "F.Cu") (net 1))
 (segment (start 107.608782 80.76625) (end 107.608782 99.81625) (width 0.2) (layer "F.Cu") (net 1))
 (segment (start 112.688782 72.035) (end 112.688782 75.68625) (width 0.2) (layer "F.Cu") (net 1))
 (segment (start 107.608782 99.81625) (end 107.608782 118.86625) (width 0.2) (layer "F.Cu") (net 1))
 (segment (start 115.387532 69.495) (end 126.658782 80.76625) (width 0.2) (layer "F.Cu") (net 3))
 (segment (start 126.658782 80.76625) (end 126.658782 99.81625) (width 0.2) (layer "F.Cu") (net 3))
 (segment (start 113.523782 69.495) (end 115.387532 69.495) (width 0.2) (layer "F.Cu") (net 3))
 (segment (start 126.658782 99.81625) (end 126.658782 118.86625) (width 0.2) (layer "F.Cu") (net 3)))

